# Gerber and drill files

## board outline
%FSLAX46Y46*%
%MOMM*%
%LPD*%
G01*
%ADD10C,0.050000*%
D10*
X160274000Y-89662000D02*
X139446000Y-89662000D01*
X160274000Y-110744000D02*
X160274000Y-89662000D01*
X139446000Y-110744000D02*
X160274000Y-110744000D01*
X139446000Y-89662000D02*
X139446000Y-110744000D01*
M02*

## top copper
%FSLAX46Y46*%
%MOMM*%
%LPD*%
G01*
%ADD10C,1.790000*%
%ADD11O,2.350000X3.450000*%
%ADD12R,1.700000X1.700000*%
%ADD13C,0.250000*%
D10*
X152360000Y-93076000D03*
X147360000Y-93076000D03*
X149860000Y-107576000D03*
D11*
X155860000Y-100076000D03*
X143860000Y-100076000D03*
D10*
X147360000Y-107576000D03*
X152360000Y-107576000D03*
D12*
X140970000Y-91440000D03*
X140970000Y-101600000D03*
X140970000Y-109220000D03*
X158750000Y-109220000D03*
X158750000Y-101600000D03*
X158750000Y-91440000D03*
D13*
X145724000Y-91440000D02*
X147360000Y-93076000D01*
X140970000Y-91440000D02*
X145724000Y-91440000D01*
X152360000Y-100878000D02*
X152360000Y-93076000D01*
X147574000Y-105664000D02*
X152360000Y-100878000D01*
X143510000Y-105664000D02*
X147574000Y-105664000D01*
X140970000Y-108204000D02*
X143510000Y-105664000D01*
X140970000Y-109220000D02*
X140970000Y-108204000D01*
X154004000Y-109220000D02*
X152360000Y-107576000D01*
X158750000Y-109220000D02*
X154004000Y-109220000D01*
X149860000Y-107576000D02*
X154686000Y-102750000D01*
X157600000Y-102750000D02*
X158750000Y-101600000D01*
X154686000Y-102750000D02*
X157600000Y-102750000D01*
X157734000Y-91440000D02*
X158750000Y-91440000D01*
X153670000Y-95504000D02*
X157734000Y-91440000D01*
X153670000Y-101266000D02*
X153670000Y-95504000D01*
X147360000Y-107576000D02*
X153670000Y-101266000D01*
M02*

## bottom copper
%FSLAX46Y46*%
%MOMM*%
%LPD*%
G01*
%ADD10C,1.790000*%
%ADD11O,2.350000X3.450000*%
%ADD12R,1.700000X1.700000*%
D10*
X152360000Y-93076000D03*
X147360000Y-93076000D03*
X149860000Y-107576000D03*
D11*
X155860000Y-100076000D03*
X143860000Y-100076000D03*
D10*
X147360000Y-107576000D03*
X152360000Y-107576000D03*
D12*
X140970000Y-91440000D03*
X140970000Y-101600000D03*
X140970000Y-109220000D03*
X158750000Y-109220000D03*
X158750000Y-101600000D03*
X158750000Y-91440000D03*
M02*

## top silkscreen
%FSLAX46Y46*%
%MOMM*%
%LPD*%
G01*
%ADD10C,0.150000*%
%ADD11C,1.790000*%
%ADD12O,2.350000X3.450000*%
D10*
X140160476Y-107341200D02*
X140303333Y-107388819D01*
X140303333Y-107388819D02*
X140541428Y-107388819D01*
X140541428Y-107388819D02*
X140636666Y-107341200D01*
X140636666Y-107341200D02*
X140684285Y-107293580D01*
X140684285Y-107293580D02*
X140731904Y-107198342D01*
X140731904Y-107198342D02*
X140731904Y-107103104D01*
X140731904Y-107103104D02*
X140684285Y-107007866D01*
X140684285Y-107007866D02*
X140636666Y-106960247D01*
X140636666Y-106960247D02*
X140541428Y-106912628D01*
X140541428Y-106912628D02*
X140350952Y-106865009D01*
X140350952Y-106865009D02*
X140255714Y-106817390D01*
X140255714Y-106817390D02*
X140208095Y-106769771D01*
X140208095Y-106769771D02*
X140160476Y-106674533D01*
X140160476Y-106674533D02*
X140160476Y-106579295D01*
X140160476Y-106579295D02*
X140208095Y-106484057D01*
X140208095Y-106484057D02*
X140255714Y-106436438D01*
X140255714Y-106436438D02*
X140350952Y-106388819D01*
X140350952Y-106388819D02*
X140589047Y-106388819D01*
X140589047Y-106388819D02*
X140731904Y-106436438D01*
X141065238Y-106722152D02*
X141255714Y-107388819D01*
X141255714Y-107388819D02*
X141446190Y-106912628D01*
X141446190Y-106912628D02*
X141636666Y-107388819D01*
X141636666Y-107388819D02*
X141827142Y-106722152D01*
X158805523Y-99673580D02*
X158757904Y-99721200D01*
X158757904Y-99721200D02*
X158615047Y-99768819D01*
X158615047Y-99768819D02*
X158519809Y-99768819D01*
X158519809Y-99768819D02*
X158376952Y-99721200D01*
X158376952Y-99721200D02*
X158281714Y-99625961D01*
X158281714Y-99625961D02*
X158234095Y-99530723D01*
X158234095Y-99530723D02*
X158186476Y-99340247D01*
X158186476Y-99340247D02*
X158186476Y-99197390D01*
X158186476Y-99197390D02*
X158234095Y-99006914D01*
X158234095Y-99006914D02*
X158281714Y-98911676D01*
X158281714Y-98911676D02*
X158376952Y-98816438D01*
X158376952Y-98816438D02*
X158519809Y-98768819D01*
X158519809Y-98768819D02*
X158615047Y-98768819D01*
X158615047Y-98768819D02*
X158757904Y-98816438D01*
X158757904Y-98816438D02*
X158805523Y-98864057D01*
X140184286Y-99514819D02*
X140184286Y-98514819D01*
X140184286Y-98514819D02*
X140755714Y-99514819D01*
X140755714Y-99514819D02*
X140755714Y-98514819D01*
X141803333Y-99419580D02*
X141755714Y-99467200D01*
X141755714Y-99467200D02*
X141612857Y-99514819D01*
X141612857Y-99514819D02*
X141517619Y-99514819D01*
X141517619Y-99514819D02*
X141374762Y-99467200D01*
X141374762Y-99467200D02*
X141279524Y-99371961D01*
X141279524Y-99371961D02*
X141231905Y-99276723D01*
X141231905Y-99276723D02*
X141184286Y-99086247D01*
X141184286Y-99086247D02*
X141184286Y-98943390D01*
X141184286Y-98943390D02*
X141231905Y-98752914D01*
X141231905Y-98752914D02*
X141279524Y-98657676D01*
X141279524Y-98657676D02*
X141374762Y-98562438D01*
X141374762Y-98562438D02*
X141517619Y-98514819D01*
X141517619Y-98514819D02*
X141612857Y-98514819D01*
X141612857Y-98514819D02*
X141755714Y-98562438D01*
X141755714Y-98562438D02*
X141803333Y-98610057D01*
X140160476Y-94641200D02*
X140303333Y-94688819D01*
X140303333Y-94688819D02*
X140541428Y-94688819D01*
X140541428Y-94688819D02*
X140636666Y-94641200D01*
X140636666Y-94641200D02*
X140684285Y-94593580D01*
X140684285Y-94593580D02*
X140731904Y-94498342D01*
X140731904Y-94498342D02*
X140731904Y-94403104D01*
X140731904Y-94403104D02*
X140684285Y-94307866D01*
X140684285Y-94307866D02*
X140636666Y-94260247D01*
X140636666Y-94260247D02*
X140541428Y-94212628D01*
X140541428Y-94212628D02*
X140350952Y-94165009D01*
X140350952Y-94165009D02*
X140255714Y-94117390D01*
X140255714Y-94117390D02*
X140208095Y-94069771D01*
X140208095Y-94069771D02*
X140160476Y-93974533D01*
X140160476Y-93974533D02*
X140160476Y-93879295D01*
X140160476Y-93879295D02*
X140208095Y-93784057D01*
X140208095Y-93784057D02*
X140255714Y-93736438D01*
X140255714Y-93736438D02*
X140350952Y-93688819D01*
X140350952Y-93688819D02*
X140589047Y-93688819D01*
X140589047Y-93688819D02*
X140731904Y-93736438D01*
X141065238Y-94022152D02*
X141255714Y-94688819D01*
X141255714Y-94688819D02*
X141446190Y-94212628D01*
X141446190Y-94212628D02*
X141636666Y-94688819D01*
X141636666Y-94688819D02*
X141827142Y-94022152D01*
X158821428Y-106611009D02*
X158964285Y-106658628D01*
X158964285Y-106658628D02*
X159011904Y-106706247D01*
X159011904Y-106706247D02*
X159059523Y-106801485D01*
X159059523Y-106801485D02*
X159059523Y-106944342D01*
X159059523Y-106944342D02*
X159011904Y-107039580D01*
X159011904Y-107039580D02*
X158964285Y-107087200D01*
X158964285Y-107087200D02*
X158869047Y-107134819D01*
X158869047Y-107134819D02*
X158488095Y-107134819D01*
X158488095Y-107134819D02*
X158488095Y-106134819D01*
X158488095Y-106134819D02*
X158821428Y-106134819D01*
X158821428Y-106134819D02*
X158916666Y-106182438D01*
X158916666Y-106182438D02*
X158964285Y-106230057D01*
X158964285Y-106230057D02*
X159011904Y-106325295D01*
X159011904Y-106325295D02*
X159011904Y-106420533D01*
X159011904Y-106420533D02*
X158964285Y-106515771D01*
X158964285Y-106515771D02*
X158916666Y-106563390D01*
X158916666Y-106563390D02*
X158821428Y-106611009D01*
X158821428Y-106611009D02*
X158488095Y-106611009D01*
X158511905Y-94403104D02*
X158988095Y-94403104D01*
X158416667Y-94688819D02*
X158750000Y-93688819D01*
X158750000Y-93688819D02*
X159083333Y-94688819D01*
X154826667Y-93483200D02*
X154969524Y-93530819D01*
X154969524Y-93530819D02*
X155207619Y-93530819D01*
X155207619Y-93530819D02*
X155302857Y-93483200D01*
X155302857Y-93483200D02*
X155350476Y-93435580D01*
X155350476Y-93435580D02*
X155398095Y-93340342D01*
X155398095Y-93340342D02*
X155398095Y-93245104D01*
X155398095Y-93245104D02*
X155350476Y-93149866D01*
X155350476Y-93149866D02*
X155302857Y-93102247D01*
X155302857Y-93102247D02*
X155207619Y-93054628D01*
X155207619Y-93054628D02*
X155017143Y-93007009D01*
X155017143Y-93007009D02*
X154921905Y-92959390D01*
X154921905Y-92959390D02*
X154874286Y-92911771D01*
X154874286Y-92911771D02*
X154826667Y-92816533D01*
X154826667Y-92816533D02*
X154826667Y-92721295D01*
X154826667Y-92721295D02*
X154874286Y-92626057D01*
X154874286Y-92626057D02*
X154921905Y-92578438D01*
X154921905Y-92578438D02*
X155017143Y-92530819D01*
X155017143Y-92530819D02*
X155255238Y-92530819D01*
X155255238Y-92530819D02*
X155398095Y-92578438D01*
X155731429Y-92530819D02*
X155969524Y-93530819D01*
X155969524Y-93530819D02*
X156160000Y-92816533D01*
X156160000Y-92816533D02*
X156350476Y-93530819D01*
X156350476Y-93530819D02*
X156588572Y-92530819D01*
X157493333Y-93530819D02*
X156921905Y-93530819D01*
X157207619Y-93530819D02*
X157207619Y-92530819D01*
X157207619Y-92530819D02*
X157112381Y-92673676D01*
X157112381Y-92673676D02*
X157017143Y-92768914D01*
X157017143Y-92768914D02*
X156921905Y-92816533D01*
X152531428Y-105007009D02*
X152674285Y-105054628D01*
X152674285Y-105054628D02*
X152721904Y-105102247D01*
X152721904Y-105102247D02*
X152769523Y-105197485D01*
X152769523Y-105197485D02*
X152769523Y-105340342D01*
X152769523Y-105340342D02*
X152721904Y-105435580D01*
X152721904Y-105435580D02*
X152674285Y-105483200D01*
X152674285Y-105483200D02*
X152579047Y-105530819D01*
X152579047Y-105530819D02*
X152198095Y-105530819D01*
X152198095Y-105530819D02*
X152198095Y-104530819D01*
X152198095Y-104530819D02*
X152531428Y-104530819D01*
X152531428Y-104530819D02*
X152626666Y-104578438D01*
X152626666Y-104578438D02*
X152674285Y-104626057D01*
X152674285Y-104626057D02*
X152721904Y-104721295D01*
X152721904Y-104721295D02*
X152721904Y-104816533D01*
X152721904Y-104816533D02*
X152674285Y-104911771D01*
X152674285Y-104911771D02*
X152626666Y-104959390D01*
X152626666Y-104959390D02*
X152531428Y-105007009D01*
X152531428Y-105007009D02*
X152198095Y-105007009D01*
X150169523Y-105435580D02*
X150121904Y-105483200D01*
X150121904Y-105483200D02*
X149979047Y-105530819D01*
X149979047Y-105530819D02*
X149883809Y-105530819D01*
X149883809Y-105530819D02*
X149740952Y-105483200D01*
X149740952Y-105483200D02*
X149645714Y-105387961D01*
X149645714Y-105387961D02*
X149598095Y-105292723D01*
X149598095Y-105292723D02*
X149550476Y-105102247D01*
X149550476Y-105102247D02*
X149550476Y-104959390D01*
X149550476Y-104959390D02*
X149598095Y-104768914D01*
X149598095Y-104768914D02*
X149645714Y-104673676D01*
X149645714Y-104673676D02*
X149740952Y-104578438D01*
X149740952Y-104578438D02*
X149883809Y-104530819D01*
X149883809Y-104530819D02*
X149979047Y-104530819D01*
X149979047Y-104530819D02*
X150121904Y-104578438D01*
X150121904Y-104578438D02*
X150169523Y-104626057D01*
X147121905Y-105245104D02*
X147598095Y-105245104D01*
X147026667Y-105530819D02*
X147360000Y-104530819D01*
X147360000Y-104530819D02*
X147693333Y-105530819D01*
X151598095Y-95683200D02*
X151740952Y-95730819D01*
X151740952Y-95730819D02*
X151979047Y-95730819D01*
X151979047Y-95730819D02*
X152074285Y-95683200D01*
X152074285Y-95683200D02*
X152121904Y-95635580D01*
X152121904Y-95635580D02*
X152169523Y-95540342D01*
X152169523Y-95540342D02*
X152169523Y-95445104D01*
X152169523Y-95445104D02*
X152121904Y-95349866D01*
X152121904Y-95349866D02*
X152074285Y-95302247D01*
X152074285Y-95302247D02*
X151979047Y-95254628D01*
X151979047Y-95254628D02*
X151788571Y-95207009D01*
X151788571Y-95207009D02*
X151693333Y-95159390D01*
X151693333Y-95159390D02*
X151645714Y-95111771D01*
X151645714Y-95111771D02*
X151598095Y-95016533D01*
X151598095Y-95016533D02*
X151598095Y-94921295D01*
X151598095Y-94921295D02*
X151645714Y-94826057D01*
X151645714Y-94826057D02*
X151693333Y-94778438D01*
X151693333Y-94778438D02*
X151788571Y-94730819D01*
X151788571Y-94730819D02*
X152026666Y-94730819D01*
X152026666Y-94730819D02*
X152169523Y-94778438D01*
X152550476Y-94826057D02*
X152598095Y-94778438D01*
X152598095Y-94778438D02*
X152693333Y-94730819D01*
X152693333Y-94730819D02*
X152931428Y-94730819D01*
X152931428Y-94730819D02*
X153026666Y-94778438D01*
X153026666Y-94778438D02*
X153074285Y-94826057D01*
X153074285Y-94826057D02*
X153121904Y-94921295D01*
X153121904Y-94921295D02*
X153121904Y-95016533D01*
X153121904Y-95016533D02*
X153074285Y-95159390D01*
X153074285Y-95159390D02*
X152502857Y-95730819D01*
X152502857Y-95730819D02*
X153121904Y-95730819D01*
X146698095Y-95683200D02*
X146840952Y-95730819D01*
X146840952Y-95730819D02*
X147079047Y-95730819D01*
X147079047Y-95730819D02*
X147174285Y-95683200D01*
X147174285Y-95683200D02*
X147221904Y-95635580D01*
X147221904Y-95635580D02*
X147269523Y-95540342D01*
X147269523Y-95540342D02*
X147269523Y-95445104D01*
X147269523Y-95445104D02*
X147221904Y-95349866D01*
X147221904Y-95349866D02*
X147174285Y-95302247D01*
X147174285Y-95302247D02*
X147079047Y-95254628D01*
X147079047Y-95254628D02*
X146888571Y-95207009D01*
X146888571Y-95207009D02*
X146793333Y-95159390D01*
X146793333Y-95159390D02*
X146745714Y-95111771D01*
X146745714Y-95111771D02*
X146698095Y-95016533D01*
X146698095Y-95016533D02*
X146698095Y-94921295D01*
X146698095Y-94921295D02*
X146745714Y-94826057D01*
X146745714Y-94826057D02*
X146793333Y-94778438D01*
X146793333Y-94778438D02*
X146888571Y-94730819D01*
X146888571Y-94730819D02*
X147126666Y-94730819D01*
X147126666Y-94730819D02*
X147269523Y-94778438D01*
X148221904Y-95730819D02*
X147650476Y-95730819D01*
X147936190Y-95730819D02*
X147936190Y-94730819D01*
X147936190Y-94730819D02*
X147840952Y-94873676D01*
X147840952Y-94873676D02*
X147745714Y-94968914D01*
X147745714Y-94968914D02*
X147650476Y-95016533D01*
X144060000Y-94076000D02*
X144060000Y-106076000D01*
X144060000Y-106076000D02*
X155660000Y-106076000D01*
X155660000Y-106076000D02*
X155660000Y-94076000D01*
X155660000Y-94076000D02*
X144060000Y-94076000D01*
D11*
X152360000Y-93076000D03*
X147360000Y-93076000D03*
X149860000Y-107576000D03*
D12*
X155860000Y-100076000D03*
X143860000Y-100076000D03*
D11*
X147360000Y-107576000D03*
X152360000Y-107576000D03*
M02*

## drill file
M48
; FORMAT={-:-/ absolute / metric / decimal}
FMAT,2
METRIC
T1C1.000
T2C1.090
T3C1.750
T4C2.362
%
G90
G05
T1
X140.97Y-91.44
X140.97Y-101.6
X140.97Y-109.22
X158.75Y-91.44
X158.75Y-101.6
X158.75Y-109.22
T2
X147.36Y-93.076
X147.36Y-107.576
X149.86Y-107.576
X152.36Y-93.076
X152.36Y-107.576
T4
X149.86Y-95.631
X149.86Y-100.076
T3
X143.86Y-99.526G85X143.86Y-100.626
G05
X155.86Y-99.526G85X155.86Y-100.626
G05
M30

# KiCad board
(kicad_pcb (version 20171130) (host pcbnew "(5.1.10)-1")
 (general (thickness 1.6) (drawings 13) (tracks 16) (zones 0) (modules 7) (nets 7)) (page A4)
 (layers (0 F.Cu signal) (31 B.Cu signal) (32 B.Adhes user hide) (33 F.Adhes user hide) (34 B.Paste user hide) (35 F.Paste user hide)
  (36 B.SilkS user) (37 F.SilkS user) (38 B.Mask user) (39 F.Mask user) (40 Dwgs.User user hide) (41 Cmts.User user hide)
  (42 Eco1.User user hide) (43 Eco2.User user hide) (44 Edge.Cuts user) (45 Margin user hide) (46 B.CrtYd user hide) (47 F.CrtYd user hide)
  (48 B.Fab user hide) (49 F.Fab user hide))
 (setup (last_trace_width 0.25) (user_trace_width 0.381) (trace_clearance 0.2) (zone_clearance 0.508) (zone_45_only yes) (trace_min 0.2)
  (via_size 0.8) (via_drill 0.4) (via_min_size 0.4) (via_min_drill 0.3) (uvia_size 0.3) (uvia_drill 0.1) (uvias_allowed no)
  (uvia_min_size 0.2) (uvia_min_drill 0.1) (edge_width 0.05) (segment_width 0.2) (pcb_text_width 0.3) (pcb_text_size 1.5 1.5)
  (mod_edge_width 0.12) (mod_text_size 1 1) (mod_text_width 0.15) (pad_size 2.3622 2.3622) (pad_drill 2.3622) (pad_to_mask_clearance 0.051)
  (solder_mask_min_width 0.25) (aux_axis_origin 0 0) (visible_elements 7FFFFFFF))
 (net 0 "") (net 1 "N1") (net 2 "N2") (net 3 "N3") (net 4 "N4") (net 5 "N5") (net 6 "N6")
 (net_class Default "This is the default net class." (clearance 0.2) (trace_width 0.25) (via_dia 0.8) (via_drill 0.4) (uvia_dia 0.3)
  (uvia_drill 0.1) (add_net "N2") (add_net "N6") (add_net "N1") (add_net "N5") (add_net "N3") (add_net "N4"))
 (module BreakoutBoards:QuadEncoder (layer F.Cu) (at 149.86 100.076)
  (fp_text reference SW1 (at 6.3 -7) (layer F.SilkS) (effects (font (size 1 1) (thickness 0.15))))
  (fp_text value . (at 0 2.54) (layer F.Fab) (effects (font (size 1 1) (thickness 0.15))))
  (fp_line (start -5.8 -6) (end -5.8 6) (layer F.SilkS) (width 0.15))
  (fp_line (start -5.8 6) (end 5.8 6) (layer F.SilkS) (width 0.15))
  (fp_line (start 5.8 6) (end 5.8 -6) (layer F.SilkS) (width 0.15))
  (fp_line (start 5.8 -6) (end -5.8 -6) (layer F.SilkS) (width 0.15))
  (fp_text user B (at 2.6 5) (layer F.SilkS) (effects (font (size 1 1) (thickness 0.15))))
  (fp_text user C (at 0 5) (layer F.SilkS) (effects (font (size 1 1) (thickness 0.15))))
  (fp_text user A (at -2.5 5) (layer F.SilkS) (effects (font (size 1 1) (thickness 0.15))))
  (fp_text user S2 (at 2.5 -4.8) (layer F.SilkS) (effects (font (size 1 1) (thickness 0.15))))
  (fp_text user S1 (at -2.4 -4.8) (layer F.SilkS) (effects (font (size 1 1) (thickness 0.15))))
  (pad S2 thru_hole circle (at 2.5 -7) (size 1.79 1.79) (drill 1.09) (layers *.Cu *.Mask F.SilkS) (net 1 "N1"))
  (pad S1 thru_hole circle (at -2.5 -7) (size 1.79 1.79) (drill 1.09) (layers *.Cu *.Mask F.SilkS) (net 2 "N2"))
  (pad C thru_hole circle (at 0 7.5) (size 1.79 1.79) (drill 1.09) (layers *.Cu *.Mask F.SilkS) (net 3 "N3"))
  (pad 7 thru_hole oval (at 6 0) (size 2.35 3.45) (drill oval 1.75 2.85) (layers *.Cu *.Mask F.SilkS))
  (pad 6 thru_hole oval (at -6 0) (size 2.35 3.45) (drill oval 1.75 2.85) (layers *.Cu *.Mask F.SilkS))
  (pad A thru_hole circle (at -2.5 7.5) (size 1.79 1.79) (drill 1.09) (layers *.Cu *.Mask F.SilkS) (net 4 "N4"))
  (pad B thru_hole circle (at 2.5 7.5) (size 1.79 1.79) (drill 1.09) (layers *.Cu *.Mask F.SilkS) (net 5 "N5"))
  (pad "" np_thru_hole circle (at 0 0) (size 2.3622 2.3622) (drill 2.3622) (layers *.Cu *.Mask))
  (pad "" np_thru_hole circle (at 0 -4.445) (size 2.3622 2.3622) (drill 2.3622) (layers *.Cu *.Mask)))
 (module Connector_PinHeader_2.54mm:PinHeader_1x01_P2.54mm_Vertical (layer B.Cu) (at 140.97 91.44)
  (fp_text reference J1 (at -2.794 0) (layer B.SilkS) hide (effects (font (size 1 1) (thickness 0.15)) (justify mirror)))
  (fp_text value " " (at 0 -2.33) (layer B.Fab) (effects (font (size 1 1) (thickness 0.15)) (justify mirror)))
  (pad 1 thru_hole rect (at 0 0) (size 1.7 1.7) (drill 1) (layers *.Cu *.Mask) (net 2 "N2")))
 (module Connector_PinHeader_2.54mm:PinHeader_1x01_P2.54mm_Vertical (layer B.Cu) (at 140.97 101.6)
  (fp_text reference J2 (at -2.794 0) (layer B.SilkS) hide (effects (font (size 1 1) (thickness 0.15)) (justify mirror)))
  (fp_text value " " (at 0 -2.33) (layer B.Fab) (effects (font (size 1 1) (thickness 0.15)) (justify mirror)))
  (pad 1 thru_hole rect (at 0 0) (size 1.7 1.7) (drill 1) (layers *.Cu *.Mask) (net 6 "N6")))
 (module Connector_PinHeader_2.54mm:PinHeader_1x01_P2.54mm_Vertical (layer B.Cu) (at 140.97 109.22)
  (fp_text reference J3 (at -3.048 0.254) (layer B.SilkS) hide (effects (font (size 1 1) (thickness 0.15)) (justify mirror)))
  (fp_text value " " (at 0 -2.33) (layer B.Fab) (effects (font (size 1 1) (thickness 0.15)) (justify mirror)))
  (pad 1 thru_hole rect (at 0 0) (size 1.7 1.7) (drill 1) (layers *.Cu *.Mask) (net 1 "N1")))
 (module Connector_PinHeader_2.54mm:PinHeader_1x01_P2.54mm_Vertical (layer B.Cu) (at 158.75 109.22)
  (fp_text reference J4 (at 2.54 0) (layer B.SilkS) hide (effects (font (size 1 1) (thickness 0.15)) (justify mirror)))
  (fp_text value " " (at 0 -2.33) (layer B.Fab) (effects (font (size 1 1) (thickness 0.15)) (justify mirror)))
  (pad 1 thru_hole rect (at 0 0) (size 1.7 1.7) (drill 1) (layers *.Cu *.Mask) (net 5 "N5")))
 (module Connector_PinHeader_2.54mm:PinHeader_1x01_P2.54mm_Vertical (layer B.Cu) (at 158.75 101.6)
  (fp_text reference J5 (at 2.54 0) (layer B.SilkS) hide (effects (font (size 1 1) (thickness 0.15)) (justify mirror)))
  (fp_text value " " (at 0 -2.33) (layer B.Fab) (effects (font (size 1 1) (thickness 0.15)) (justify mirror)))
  (pad 1 thru_hole rect (at 0 0) (size 1.7 1.7) (drill 1) (layers *.Cu *.Mask) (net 3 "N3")))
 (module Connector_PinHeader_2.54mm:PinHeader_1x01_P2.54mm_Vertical (layer B.Cu) (at 158.75 91.44)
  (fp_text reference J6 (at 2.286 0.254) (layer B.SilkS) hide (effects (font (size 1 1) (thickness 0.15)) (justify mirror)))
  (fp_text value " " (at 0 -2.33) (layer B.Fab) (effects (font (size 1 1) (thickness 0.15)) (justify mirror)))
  (pad 1 thru_hole rect (at 0 0) (size 1.7 1.7) (drill 1) (layers *.Cu *.Mask) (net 4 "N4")))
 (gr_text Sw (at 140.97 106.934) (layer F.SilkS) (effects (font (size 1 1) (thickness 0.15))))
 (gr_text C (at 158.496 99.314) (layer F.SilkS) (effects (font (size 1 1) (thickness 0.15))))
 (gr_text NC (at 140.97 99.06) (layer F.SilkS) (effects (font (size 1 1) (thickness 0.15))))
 (gr_line (start 160.274 89.662) (end 139.446 89.662) (layer Edge.Cuts) (width 0.05))
 (gr_line (start 160.274 110.744) (end 160.274 89.662) (layer Edge.Cuts) (width 0.05))
 (gr_line (start 139.446 110.744) (end 160.274 110.744) (layer Edge.Cuts) (width 0.05))
 (gr_line (start 139.446 89.662) (end 139.446 110.744) (layer Edge.Cuts) (width 0.05))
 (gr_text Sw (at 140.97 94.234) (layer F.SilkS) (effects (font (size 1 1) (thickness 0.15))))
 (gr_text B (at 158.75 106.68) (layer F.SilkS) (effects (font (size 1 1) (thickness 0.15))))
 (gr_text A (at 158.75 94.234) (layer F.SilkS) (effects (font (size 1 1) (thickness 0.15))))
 (segment (start 145.724 91.44) (end 147.36 93.076) (width 0.25) (layer F.Cu) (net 2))
 (segment (start 140.97 91.44) (end 145.724 91.44) (width 0.25) (layer F.Cu) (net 2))
 (segment (start 152.36 100.878) (end 152.36 93.076) (width 0.25) (layer F.Cu) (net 1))
 (segment (start 147.574 105.664) (end 152.36 100.878) (width 0.25) (layer F.Cu) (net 1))
 (segment (start 143.51 105.664) (end 147.574 105.664) (width 0.25) (layer F.Cu) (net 1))
 (segment (start 140.97 108.204) (end 143.51 105.664) (width 0.25) (layer F.Cu) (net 1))
 (segment (start 140.97 109.22) (end 140.97 108.204) (width 0.25) (layer F.Cu) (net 1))
 (segment (start 154.004 109.22) (end 152.36 107.576) (width 0.25) (layer F.Cu) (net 5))
 (segment (start 158.75 109.22) (end 154.004 109.22) (width 0.25) (layer F.Cu) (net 5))
 (segment (start 149.86 107.576) (end 154.686 102.75) (width 0.25) (layer F.Cu) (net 3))
 (segment (start 157.6 102.75) (end 158.75 101.6) (width 0.25) (layer F.Cu) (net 3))
 (segment (start 154.686 102.75) (end 157.6 102.75) (width 0.25) (layer F.Cu) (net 3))
 (segment (start 157.734 91.44) (end 158.75 91.44) (width 0.25) (layer F.Cu) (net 4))
 (segment (start 153.67 95.504) (end 157.734 91.44) (width 0.25) (layer F.Cu) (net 4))
 (segment (start 153.67 101.266) (end 153.67 95.504) (width 0.25) (layer F.Cu) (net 4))
 (segment (start 147.36 107.576) (end 153.67 101.266) (width 0.25) (layer F.Cu) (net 4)))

